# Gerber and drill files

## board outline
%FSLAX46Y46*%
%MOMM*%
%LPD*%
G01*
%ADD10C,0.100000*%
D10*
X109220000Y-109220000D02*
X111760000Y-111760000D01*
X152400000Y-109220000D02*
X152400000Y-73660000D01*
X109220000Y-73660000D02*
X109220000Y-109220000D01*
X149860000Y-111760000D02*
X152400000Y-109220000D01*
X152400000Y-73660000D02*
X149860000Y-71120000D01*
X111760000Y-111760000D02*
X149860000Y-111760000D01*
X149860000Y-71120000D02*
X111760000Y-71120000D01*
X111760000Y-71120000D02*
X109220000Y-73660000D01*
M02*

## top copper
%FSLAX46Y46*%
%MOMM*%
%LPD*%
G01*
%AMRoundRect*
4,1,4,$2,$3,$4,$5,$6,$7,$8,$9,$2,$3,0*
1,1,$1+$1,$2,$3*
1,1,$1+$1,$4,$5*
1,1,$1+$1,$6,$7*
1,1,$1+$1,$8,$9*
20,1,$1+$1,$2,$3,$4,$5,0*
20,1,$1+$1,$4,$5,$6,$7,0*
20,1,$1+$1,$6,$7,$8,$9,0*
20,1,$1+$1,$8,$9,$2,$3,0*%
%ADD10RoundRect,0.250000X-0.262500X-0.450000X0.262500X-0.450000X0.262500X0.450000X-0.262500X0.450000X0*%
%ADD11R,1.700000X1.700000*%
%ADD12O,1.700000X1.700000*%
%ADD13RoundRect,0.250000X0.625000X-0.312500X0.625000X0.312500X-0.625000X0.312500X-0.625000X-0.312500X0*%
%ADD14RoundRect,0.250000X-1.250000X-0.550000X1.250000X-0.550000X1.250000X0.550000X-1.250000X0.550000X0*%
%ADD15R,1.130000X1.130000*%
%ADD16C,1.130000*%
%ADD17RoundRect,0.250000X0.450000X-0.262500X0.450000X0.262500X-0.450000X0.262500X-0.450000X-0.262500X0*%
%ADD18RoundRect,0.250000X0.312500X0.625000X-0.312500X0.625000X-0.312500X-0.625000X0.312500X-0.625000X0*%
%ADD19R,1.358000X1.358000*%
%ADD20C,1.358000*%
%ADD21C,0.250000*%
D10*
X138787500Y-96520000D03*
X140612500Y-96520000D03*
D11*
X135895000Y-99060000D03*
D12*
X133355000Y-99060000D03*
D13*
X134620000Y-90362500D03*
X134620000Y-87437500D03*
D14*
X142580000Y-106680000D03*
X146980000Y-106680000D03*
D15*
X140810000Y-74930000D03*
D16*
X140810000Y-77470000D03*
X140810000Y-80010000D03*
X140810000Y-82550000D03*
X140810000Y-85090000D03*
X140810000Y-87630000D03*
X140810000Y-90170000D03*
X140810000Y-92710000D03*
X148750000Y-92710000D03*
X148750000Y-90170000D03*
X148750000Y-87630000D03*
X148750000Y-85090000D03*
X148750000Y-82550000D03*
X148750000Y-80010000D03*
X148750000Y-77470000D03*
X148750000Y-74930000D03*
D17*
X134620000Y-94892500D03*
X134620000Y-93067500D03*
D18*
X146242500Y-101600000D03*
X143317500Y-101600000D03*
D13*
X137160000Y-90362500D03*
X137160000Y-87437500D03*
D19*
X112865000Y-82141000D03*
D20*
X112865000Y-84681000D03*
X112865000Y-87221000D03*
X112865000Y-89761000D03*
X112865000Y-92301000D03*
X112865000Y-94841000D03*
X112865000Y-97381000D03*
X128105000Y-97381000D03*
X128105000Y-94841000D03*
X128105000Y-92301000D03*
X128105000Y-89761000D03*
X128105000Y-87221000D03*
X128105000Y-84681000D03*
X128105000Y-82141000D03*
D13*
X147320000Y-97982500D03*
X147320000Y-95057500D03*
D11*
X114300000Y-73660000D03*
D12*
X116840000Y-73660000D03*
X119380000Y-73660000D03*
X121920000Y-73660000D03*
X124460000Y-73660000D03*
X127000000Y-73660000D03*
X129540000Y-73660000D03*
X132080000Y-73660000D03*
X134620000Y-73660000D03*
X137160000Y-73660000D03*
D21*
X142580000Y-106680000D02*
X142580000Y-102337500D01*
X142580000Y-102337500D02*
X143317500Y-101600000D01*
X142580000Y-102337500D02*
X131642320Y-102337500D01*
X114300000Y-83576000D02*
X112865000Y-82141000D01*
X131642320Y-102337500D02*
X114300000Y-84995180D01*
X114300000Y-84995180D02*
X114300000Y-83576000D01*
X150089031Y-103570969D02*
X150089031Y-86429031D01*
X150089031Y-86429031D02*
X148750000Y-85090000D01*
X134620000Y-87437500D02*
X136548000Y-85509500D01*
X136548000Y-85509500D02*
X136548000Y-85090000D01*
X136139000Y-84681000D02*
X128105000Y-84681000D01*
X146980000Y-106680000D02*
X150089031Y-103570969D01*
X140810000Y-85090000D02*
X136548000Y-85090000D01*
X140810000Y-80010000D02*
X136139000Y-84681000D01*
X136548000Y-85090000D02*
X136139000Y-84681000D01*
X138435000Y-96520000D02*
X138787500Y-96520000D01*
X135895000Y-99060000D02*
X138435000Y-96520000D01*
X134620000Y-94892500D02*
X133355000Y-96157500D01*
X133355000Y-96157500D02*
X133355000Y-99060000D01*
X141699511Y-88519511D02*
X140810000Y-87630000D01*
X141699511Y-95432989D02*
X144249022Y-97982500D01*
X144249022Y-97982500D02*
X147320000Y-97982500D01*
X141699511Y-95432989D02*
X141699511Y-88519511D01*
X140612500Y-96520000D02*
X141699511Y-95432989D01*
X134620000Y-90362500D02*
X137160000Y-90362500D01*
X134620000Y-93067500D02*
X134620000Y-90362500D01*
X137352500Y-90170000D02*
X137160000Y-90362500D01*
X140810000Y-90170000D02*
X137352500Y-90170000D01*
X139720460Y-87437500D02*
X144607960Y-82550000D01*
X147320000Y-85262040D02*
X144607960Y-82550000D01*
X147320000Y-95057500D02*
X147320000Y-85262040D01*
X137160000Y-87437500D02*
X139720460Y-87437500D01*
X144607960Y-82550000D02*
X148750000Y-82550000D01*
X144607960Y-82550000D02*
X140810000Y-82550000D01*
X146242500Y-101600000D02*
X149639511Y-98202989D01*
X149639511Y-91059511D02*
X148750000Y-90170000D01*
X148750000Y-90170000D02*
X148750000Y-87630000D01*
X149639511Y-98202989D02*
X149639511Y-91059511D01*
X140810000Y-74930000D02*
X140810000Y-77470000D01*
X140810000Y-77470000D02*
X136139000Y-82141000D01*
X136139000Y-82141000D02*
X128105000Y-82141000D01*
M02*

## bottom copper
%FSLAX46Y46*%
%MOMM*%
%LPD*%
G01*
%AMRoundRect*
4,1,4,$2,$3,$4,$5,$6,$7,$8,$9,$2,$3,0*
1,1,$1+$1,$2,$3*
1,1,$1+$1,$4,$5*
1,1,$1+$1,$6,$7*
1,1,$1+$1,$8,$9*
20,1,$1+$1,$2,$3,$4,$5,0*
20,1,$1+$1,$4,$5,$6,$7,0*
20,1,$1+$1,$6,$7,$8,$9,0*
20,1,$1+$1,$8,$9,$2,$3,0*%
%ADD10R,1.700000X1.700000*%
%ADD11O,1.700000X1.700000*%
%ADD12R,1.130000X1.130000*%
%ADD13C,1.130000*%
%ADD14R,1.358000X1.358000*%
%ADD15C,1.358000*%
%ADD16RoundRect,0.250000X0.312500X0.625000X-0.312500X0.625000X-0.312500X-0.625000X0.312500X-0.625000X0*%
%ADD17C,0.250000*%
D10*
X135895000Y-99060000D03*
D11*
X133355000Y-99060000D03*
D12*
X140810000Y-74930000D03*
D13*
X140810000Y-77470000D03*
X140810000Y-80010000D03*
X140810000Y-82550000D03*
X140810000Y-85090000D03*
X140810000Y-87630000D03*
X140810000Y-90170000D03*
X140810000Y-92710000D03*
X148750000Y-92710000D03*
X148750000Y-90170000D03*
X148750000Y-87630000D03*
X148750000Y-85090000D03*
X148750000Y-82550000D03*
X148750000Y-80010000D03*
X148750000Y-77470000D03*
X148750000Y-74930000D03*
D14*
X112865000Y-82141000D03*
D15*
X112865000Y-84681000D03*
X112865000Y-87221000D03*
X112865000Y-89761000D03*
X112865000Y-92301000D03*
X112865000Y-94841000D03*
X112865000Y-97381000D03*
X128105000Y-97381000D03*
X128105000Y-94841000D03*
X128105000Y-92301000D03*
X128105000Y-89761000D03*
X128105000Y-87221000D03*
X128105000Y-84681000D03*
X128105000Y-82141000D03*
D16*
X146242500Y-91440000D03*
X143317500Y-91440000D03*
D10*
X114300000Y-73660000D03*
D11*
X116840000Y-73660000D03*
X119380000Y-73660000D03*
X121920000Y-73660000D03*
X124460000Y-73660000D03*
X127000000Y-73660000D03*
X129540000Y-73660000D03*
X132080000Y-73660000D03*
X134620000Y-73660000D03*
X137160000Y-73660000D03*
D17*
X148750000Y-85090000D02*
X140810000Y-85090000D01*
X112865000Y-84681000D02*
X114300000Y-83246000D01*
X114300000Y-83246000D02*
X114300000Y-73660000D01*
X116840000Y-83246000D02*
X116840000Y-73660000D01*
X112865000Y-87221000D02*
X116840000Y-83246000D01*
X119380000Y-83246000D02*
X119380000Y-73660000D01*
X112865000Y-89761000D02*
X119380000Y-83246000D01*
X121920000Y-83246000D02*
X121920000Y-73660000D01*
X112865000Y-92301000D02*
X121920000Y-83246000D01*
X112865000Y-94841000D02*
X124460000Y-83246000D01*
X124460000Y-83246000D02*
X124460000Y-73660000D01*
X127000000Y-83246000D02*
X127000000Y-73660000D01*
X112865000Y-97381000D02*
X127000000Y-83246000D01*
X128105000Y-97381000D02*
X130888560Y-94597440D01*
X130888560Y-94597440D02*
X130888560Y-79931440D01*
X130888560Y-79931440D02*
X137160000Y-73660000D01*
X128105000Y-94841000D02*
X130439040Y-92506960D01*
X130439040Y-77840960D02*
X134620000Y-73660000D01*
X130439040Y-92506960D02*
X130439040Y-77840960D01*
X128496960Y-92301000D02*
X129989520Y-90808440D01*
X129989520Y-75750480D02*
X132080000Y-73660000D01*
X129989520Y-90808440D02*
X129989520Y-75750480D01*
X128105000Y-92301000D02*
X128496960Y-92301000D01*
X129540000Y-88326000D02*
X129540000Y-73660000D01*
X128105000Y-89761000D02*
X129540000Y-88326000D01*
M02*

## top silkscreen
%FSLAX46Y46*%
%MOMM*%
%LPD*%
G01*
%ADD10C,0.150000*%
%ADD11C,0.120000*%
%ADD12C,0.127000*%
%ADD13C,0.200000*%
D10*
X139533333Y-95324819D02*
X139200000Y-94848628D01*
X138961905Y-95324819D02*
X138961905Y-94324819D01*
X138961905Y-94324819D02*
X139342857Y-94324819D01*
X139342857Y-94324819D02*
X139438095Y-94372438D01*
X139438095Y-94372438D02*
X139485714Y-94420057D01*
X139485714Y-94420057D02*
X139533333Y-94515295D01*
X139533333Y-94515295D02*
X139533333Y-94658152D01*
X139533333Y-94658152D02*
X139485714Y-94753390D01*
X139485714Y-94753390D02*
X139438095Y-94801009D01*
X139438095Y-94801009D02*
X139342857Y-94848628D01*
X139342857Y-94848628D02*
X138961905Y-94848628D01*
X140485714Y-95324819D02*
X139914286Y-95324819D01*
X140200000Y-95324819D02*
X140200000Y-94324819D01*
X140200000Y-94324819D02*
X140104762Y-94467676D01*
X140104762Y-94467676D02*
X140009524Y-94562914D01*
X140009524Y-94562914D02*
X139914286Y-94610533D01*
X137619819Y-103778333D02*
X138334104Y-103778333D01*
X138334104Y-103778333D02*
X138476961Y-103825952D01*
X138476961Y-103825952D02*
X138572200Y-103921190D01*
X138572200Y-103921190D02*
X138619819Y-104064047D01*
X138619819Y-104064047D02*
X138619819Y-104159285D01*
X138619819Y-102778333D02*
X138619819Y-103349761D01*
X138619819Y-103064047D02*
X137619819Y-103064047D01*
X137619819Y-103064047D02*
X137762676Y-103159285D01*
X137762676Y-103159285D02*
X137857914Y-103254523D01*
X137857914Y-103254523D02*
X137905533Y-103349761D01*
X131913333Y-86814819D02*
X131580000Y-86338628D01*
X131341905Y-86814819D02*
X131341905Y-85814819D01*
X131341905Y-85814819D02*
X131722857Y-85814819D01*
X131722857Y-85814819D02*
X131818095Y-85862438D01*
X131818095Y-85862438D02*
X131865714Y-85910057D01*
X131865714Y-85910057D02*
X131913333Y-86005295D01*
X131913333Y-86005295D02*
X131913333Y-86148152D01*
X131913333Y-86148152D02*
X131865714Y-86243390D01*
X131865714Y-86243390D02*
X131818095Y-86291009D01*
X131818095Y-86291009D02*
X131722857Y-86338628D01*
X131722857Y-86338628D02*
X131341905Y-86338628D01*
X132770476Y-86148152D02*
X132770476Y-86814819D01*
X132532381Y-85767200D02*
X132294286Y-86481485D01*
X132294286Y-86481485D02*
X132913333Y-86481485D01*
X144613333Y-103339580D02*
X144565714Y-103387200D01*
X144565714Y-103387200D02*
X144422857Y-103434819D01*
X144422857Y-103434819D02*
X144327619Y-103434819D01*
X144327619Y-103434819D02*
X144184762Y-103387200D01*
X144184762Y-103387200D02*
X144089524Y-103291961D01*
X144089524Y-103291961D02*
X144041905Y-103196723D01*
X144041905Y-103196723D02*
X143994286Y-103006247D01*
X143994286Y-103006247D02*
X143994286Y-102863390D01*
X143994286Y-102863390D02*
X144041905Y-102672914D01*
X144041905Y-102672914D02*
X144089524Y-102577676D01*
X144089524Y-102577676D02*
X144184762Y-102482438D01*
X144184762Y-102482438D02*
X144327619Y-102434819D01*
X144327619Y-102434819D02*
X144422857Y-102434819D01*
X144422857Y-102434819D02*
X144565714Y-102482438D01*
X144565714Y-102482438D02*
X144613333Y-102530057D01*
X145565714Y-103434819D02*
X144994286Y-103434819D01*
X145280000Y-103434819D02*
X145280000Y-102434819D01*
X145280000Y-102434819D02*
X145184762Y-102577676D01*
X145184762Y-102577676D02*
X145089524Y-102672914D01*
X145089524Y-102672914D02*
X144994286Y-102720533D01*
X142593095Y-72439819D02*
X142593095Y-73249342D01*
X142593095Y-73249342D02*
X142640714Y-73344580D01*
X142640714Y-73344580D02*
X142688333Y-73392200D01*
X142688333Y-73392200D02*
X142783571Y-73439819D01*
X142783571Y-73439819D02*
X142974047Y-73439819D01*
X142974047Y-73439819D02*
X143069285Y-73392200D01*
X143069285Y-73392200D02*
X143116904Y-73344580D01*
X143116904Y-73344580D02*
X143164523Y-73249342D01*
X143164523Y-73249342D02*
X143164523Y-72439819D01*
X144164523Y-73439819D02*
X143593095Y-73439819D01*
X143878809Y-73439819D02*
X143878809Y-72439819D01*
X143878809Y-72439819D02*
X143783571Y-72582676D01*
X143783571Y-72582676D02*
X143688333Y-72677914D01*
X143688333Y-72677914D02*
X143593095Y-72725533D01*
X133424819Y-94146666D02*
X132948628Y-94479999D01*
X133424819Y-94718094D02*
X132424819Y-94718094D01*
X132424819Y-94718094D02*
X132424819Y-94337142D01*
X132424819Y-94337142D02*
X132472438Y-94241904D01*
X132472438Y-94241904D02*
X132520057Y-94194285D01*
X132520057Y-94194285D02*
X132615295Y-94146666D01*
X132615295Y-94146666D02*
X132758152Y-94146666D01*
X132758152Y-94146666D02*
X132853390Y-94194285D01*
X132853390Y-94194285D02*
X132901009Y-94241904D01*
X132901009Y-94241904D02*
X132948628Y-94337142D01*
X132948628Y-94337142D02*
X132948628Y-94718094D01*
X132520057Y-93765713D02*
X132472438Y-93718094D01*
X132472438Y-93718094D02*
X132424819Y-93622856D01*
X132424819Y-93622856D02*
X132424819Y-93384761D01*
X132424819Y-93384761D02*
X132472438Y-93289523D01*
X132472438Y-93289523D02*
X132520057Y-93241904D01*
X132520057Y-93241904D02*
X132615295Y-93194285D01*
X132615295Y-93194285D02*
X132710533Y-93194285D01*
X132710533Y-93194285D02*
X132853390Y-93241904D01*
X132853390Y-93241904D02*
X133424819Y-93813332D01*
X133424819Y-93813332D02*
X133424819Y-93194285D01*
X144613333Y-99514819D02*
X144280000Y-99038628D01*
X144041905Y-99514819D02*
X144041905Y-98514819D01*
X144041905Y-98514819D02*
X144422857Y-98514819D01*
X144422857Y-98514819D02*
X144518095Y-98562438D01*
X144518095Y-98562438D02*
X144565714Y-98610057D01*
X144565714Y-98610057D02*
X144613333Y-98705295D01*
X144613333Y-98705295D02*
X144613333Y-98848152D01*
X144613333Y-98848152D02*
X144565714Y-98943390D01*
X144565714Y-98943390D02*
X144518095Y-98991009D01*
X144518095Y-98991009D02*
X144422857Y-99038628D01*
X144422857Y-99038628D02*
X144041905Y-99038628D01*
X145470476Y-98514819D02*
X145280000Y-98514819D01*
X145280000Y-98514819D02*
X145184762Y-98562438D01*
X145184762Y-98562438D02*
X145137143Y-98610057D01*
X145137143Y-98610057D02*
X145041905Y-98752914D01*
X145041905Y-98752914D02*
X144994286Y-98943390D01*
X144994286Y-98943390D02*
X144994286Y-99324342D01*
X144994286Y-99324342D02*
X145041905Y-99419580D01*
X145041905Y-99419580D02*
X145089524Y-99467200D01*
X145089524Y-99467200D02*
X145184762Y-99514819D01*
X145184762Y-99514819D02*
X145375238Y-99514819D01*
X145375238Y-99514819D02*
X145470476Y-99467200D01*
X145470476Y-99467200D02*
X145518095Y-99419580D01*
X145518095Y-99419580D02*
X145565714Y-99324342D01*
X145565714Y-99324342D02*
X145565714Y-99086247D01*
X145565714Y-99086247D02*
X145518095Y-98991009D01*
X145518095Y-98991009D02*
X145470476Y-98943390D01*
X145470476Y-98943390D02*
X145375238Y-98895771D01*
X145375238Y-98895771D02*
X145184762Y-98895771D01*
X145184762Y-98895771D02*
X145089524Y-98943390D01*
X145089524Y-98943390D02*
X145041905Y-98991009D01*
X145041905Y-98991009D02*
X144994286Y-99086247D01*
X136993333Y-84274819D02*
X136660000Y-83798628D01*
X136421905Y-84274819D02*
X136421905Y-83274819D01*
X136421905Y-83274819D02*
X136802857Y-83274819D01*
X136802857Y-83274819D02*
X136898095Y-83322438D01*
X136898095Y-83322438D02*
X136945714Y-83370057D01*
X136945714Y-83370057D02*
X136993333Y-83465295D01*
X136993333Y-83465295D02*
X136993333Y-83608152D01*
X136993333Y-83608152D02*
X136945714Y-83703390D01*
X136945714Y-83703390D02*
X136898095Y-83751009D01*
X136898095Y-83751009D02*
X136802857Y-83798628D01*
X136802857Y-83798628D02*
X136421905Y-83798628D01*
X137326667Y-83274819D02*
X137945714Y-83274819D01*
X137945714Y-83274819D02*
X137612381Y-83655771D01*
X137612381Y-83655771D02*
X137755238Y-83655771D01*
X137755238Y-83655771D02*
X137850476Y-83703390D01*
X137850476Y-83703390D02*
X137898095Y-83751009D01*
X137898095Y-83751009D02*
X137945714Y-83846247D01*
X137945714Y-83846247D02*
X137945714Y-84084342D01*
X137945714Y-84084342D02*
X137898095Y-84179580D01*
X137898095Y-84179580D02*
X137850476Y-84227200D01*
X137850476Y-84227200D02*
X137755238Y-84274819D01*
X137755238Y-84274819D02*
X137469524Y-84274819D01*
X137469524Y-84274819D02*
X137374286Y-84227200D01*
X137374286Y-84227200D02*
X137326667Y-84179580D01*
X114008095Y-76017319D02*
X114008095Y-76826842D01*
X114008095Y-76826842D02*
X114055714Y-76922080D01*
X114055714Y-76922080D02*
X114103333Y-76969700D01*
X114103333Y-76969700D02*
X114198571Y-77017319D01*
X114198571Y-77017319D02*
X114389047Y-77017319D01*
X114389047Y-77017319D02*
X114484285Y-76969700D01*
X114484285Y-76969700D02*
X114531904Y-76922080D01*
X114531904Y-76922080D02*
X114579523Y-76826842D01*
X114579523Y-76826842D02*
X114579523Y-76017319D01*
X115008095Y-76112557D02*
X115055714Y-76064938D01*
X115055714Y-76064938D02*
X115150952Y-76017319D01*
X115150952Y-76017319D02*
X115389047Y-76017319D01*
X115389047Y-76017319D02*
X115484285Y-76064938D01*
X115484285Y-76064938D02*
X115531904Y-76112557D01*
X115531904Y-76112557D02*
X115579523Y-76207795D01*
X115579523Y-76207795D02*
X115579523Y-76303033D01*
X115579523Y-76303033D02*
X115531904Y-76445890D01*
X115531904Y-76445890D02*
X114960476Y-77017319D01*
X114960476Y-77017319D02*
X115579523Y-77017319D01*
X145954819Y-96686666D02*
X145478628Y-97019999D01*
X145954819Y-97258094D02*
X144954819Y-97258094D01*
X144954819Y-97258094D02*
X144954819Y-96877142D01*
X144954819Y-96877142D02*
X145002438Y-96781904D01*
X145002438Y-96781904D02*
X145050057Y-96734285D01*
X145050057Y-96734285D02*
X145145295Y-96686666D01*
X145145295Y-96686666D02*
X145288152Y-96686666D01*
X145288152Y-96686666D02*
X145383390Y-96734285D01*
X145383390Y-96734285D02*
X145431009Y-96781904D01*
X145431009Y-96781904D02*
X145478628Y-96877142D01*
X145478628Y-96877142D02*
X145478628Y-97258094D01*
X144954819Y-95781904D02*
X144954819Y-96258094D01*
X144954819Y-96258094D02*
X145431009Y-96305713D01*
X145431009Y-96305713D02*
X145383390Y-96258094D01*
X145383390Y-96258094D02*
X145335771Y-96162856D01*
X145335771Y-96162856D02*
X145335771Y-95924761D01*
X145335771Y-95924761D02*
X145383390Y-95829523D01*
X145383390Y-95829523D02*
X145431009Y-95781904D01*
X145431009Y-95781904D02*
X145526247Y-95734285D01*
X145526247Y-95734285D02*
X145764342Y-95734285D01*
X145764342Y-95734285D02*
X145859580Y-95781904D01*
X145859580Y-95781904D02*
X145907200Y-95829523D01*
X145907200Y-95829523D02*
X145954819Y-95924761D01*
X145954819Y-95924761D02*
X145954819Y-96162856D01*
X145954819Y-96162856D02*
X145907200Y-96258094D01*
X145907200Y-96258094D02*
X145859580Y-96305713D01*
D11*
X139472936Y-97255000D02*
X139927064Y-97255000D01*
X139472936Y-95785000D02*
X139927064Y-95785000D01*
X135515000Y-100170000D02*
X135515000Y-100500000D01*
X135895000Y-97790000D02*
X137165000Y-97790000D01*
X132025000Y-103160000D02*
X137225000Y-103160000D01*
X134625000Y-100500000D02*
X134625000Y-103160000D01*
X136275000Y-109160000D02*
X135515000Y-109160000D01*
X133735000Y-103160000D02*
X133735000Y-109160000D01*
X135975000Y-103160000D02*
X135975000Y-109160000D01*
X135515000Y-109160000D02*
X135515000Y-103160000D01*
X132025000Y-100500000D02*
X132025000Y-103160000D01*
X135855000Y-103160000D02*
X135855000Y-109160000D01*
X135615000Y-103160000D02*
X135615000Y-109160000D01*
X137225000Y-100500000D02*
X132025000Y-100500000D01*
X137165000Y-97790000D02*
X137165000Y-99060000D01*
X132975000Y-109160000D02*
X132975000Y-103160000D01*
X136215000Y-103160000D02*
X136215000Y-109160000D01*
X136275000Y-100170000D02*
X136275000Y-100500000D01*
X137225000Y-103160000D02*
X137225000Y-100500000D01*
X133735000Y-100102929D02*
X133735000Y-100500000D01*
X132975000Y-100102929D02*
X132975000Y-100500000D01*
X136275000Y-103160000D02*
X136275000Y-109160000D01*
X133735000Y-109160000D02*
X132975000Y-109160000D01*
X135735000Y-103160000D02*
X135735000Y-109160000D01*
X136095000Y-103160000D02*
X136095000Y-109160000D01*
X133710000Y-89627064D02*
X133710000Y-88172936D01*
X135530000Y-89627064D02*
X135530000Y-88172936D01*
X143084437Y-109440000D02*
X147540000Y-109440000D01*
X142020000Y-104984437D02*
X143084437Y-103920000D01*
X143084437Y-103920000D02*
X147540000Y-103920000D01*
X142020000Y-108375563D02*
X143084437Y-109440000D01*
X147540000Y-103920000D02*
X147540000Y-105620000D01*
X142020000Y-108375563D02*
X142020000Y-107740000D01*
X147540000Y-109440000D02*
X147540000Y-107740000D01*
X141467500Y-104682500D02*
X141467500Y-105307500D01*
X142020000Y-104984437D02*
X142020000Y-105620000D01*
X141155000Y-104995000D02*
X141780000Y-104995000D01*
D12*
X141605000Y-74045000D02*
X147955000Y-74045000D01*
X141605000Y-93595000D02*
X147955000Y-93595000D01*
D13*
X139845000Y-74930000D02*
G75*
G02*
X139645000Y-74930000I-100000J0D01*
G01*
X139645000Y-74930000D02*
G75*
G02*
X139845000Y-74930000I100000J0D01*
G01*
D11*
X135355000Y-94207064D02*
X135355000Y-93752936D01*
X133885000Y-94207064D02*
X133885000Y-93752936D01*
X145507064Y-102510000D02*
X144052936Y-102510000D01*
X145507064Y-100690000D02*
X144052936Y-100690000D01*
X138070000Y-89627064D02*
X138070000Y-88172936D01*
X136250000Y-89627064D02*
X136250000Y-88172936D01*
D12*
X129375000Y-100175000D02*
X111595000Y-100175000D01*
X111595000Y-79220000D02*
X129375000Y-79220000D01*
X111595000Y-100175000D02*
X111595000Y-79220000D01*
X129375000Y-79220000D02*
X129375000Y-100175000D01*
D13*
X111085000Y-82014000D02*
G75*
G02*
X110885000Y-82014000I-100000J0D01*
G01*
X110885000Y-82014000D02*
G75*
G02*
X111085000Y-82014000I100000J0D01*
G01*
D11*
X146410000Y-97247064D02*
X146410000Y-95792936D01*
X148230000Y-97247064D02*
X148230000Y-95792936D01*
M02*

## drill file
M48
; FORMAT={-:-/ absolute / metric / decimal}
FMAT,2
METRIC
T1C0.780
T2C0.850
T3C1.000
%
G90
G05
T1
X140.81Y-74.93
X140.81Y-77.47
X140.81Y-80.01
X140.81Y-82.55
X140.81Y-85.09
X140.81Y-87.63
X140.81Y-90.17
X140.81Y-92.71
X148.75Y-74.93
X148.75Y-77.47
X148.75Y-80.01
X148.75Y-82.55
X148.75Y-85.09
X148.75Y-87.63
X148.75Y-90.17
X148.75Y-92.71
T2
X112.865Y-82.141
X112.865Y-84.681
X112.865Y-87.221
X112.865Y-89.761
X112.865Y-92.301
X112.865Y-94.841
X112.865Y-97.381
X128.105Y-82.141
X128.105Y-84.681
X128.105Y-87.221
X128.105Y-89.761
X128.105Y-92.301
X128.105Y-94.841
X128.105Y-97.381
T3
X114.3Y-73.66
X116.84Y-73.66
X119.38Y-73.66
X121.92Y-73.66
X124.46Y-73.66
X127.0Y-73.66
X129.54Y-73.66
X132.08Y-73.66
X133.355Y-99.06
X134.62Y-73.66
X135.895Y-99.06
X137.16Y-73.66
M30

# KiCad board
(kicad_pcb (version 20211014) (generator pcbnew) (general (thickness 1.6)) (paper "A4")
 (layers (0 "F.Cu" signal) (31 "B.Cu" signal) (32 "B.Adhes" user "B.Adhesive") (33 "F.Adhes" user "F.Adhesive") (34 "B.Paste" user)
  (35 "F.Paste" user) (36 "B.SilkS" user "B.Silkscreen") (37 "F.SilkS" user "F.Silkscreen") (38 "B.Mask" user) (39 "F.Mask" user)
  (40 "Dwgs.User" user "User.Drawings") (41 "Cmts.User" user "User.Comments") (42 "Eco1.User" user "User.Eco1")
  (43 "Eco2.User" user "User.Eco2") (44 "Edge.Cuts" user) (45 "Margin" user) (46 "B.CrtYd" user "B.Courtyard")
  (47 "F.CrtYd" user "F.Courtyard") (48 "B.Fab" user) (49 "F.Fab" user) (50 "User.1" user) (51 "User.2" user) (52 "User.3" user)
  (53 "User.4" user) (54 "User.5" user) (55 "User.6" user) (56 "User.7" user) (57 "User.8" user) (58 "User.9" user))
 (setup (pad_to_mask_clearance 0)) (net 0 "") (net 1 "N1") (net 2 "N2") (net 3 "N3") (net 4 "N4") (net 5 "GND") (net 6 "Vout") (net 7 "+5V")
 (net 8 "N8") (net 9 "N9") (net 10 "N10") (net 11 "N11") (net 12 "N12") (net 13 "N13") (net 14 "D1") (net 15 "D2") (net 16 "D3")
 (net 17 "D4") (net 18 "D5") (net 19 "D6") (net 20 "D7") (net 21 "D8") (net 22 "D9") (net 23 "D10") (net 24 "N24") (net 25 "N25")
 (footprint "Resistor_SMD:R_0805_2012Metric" (layer "F.Cu") (at 139.7 96.52)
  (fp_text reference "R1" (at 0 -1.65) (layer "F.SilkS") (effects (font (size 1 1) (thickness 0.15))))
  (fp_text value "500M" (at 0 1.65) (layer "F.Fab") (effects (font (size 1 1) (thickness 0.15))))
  (fp_line (start -0.227064 0.735) (end 0.227064 0.735) (layer "F.SilkS") (width 0.12))
  (fp_line (start -0.227064 -0.735) (end 0.227064 -0.735) (layer "F.SilkS") (width 0.12))
  (pad "1" smd roundrect (at -0.9125 0) (size 1.025 1.4) (layers "F.Cu" "F.Paste" "F.Mask") (roundrect_rratio 0.243902) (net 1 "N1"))
  (pad "2" smd roundrect (at 0.9125 0) (size 1.025 1.4) (layers "F.Cu" "F.Paste" "F.Mask") (roundrect_rratio 0.243902) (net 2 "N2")))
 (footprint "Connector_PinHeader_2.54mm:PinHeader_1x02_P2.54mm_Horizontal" (layer "F.Cu") (at 135.895 99.06 -90)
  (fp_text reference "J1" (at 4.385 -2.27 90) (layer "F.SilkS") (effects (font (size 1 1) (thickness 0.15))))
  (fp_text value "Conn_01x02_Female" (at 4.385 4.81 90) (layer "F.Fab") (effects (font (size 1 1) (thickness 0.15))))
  (fp_line (start 1.11 0.38) (end 1.44 0.38) (layer "F.SilkS") (width 0.12))
  (fp_line (start -1.27 0) (end -1.27 -1.27) (layer "F.SilkS") (width 0.12))
  (fp_line (start 4.1 3.87) (end 4.1 -1.33) (layer "F.SilkS") (width 0.12))
  (fp_line (start 1.44 1.27) (end 4.1 1.27) (layer "F.SilkS") (width 0.12))
  (fp_line (start 10.1 -0.38) (end 10.1 0.38) (layer "F.SilkS") (width 0.12))
  (fp_line (start 4.1 2.16) (end 10.1 2.16) (layer "F.SilkS") (width 0.12))
  (fp_line (start 4.1 -0.08) (end 10.1 -0.08) (layer "F.SilkS") (width 0.12))
  (fp_line (start 10.1 0.38) (end 4.1 0.38) (layer "F.SilkS") (width 0.12))
  (fp_line (start 1.44 3.87) (end 4.1 3.87) (layer "F.SilkS") (width 0.12))
  (fp_line (start 4.1 0.04) (end 10.1 0.04) (layer "F.SilkS") (width 0.12))
  (fp_line (start 4.1 0.28) (end 10.1 0.28) (layer "F.SilkS") (width 0.12))
  (fp_line (start 1.44 -1.33) (end 1.44 3.87) (layer "F.SilkS") (width 0.12))
  (fp_line (start -1.27 -1.27) (end 0 -1.27) (layer "F.SilkS") (width 0.12))
  (fp_line (start 10.1 2.92) (end 4.1 2.92) (layer "F.SilkS") (width 0.12))
  (fp_line (start 4.1 -0.32) (end 10.1 -0.32) (layer "F.SilkS") (width 0.12))
  (fp_line (start 1.11 -0.38) (end 1.44 -0.38) (layer "F.SilkS") (width 0.12))
  (fp_line (start 4.1 -1.33) (end 1.44 -1.33) (layer "F.SilkS") (width 0.12))
  (fp_line (start 1.042929 2.16) (end 1.44 2.16) (layer "F.SilkS") (width 0.12))
  (fp_line (start 1.042929 2.92) (end 1.44 2.92) (layer "F.SilkS") (width 0.12))
  (fp_line (start 4.1 -0.38) (end 10.1 -0.38) (layer "F.SilkS") (width 0.12))
  (fp_line (start 10.1 2.16) (end 10.1 2.92) (layer "F.SilkS") (width 0.12))
  (fp_line (start 4.1 0.16) (end 10.1 0.16) (layer "F.SilkS") (width 0.12))
  (fp_line (start 4.1 -0.2) (end 10.1 -0.2) (layer "F.SilkS") (width 0.12))
  (pad "1" thru_hole rect (at 0 0 270) (size 1.7 1.7) (drill 1) (layers *.Cu *.Mask) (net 1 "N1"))
  (pad "2" thru_hole oval (at 0 2.54 270) (size 1.7 1.7) (drill 1) (layers *.Cu *.Mask) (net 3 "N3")))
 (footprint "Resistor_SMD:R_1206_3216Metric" (layer "F.Cu") (at 134.62 88.9 90)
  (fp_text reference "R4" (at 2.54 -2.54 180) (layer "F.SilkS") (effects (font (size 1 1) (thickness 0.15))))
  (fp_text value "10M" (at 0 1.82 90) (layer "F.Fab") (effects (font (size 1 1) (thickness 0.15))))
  (fp_line (start -0.727064 -0.91) (end 0.727064 -0.91) (layer "F.SilkS") (width 0.12))
  (fp_line (start -0.727064 0.91) (end 0.727064 0.91) (layer "F.SilkS") (width 0.12))
  (pad "1" smd roundrect (at -1.4625 0 90) (size 1.125 1.75) (layers "F.Cu" "F.Paste" "F.Mask") (roundrect_rratio 0.222222) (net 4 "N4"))
  (pad "2" smd roundrect (at 1.4625 0 90) (size 1.125 1.75) (layers "F.Cu" "F.Paste" "F.Mask") (roundrect_rratio 0.222222) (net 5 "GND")))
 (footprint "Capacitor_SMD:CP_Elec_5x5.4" (layer "F.Cu") (at 144.78 106.68)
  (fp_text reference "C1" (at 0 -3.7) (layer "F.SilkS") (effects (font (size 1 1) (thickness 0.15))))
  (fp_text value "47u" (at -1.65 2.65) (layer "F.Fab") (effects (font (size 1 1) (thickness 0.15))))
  (fp_line (start -1.695563 2.76) (end 2.76 2.76) (layer "F.SilkS") (width 0.12))
  (fp_line (start -2.76 -1.695563) (end -1.695563 -2.76) (layer "F.SilkS") (width 0.12))
  (fp_line (start -1.695563 -2.76) (end 2.76 -2.76) (layer "F.SilkS") (width 0.12))
  (fp_line (start -2.76 1.695563) (end -1.695563 2.76) (layer "F.SilkS") (width 0.12))
  (fp_line (start 2.76 -2.76) (end 2.76 -1.06) (layer "F.SilkS") (width 0.12))
  (fp_line (start -2.76 1.695563) (end -2.76 1.06) (layer "F.SilkS") (width 0.12))
  (fp_line (start 2.76 2.76) (end 2.76 1.06) (layer "F.SilkS") (width 0.12))
  (fp_line (start -3.3125 -1.9975) (end -3.3125 -1.3725) (layer "F.SilkS") (width 0.12))
  (fp_line (start -2.76 -1.695563) (end -2.76 -1.06) (layer "F.SilkS") (width 0.12))
  (fp_line (start -3.625 -1.685) (end -3 -1.685) (layer "F.SilkS") (width 0.12))
  (pad "1" smd roundrect (at -2.2 0) (size 3 1.6) (layers "F.Cu" "F.Paste" "F.Mask") (roundrect_rratio 0.15625) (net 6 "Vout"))
  (pad "2" smd roundrect (at 2.2 0) (size 3 1.6) (layers "F.Cu" "F.Paste" "F.Mask") (roundrect_rratio 0.15625) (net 5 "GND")))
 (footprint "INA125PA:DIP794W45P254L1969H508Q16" (layer "F.Cu") (at 144.78 83.82)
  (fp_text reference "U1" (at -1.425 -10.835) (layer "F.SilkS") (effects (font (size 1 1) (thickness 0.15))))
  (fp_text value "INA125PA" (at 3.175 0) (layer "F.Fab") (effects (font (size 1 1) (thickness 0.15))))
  (fp_line (start -3.175 -9.775) (end 3.175 -9.775) (layer "F.SilkS") (width 0.127))
  (fp_line (start -3.175 9.775) (end 3.175 9.775) (layer "F.SilkS") (width 0.127))
  (fp_circle (center -5.035 -8.89) (end -4.935 -8.89) (layer "F.SilkS") (width 0.2) (fill none))
  (pad "1" thru_hole rect locked (at -3.97 -8.89) (size 1.13 1.13) (drill 0.78) (layers *.Cu *.Mask) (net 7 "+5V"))
  (pad "2" thru_hole circle locked (at -3.97 -6.35) (size 1.13 1.13) (drill 0.78) (layers *.Cu *.Mask) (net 7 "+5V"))
  (pad "3" thru_hole circle locked (at -3.97 -3.81) (size 1.13 1.13) (drill 0.78) (layers *.Cu *.Mask) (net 5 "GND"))
  (pad "4" thru_hole circle locked (at -3.97 -1.27) (size 1.13 1.13) (drill 0.78) (layers *.Cu *.Mask) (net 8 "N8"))
  (pad "5" thru_hole circle locked (at -3.97 1.27) (size 1.13 1.13) (drill 0.78) (layers *.Cu *.Mask) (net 5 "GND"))
  (pad "6" thru_hole circle locked (at -3.97 3.81) (size 1.13 1.13) (drill 0.78) (layers *.Cu *.Mask) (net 2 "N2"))
  (pad "7" thru_hole circle locked (at -3.97 6.35) (size 1.13 1.13) (drill 0.78) (layers *.Cu *.Mask) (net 4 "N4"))
  (pad "8" thru_hole circle locked (at -3.97 8.89) (size 1.13 1.13) (drill 0.78) (layers *.Cu *.Mask) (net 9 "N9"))
  (pad "9" thru_hole circle locked (at 3.97 8.89) (size 1.13 1.13) (drill 0.78) (layers *.Cu *.Mask) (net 9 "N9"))
  (pad "10" thru_hole circle locked (at 3.97 6.35) (size 1.13 1.13) (drill 0.78) (layers *.Cu *.Mask) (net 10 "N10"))
  (pad "11" thru_hole circle locked (at 3.97 3.81) (size 1.13 1.13) (drill 0.78) (layers *.Cu *.Mask) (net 10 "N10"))
  (pad "12" thru_hole circle locked (at 3.97 1.27) (size 1.13 1.13) (drill 0.78) (layers *.Cu *.Mask) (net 5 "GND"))
  (pad "13" thru_hole circle locked (at 3.97 -1.27) (size 1.13 1.13) (drill 0.78) (layers *.Cu *.Mask) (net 8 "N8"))
  (pad "14" thru_hole circle locked (at 3.97 -3.81) (size 1.13 1.13) (drill 0.78) (layers *.Cu *.Mask) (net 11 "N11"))
  (pad "15" thru_hole circle locked (at 3.97 -6.35) (size 1.13 1.13) (drill 0.78) (layers *.Cu *.Mask) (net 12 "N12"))
  (pad "16" thru_hole circle locked (at 3.97 -8.89) (size 1.13 1.13) (drill 0.78) (layers *.Cu *.Mask) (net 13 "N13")))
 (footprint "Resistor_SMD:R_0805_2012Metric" (layer "F.Cu") (at 134.62 93.98 90)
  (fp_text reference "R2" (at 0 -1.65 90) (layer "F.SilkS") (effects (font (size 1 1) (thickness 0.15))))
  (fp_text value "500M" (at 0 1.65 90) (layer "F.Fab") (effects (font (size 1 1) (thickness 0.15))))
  (fp_line (start -0.227064 0.735) (end 0.227064 0.735) (layer "F.SilkS") (width 0.12))
  (fp_line (start -0.227064 -0.735) (end 0.227064 -0.735) (layer "F.SilkS") (width 0.12))
  (pad "1" smd roundrect (at -0.9125 0 90) (size 1.025 1.4) (layers "F.Cu" "F.Paste" "F.Mask") (roundrect_rratio 0.243902) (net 3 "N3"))
  (pad "2" smd roundrect (at 0.9125 0 90) (size 1.025 1.4) (layers "F.Cu" "F.Paste" "F.Mask") (roundrect_rratio 0.243902) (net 4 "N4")))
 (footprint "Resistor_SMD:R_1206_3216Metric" (layer "F.Cu") (at 144.78 101.6 180)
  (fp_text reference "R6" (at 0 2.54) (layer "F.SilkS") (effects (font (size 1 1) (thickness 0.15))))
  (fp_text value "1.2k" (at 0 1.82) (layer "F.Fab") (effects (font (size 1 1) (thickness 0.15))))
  (fp_line (start -0.727064 -0.91) (end 0.727064 -0.91) (layer "F.SilkS") (width 0.12))
  (fp_line (start -0.727064 0.91) (end 0.727064 0.91) (layer "F.SilkS") (width 0.12))
  (pad "1" smd roundrect (at -1.4625 0 180) (size 1.125 1.75) (layers "F.Cu" "F.Paste" "F.Mask") (roundrect_rratio 0.222222) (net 10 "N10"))
  (pad "2" smd roundrect (at 1.4625 0 180) (size 1.125 1.75) (layers "F.Cu" "F.Paste" "F.Mask") (roundrect_rratio 0.222222) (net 6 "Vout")))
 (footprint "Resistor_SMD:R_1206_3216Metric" (layer "F.Cu") (at 137.16 88.9 90)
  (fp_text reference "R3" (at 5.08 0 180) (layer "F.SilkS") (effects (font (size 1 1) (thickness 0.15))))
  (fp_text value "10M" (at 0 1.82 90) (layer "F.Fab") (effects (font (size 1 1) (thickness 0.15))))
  (fp_line (start -0.727064 0.91) (end 0.727064 0.91) (layer "F.SilkS") (width 0.12))
  (fp_line (start -0.727064 -0.91) (end 0.727064 -0.91) (layer "F.SilkS") (width 0.12))
  (pad "1" smd roundrect (at -1.4625 0 90) (size 1.125 1.75) (layers "F.Cu" "F.Paste" "F.Mask") (roundrect_rratio 0.222222) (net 4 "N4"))
  (pad "2" smd roundrect (at 1.4625 0 90) (size 1.125 1.75) (layers "F.Cu" "F.Paste" "F.Mask") (roundrect_rratio 0.222222) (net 8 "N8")))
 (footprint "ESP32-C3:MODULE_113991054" (layer "F.Cu") (at 120.485 89.6975)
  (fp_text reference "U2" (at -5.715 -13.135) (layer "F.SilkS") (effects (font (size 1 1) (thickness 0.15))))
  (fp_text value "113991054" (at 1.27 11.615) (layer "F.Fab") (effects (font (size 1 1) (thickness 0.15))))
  (fp_line (start 8.89 10.4775) (end -8.89 10.4775) (layer "F.SilkS") (width 0.127))
  (fp_line (start -8.89 -10.4775) (end 8.89 -10.4775) (layer "F.SilkS") (width 0.127))
  (fp_line (start -8.89 10.4775) (end -8.89 -10.4775) (layer "F.SilkS") (width 0.127))
  (fp_line (start 8.89 -10.4775) (end 8.89 10.4775) (layer "F.SilkS") (width 0.127))
  (fp_circle (center -9.5 -7.6835) (end -9.4 -7.6835) (layer "F.SilkS") (width 0.2) (fill none))
  (pad "1" thru_hole rect locked (at -7.62 -7.5565) (size 1.358 1.358) (drill 0.85) (layers *.Cu *.Mask) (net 6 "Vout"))
  (pad "2" thru_hole circle locked (at -7.62 -5.0165) (size 1.358 1.358) (drill 0.85) (layers *.Cu *.Mask) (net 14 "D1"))
  (pad "3" thru_hole circle locked (at -7.62 -2.4765) (size 1.358 1.358) (drill 0.85) (layers *.Cu *.Mask) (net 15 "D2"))
  (pad "4" thru_hole circle locked (at -7.62 0.0635) (size 1.358 1.358) (drill 0.85) (layers *.Cu *.Mask) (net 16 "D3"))
  (pad "5" thru_hole circle locked (at -7.62 2.6035) (size 1.358 1.358) (drill 0.85) (layers *.Cu *.Mask) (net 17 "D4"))
  (pad "6" thru_hole circle locked (at -7.62 5.1435) (size 1.358 1.358) (drill 0.85) (layers *.Cu *.Mask) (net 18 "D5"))
  (pad "7" thru_hole circle locked (at -7.62 7.6835) (size 1.358 1.358) (drill 0.85) (layers *.Cu *.Mask) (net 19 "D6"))
  (pad "8" thru_hole circle locked (at 7.62 7.6835) (size 1.358 1.358) (drill 0.85) (layers *.Cu *.Mask) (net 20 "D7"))
  (pad "9" thru_hole circle locked (at 7.62 5.1435) (size 1.358 1.358) (drill 0.85) (layers *.Cu *.Mask) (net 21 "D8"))
  (pad "10" thru_hole circle locked (at 7.62 2.6035) (size 1.358 1.358) (drill 0.85) (layers *.Cu *.Mask) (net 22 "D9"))
  (pad "11" thru_hole circle locked (at 7.62 0.0635) (size 1.358 1.358) (drill 0.85) (layers *.Cu *.Mask) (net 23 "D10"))
  (pad "12" thru_hole circle locked (at 7.62 -2.4765) (size 1.358 1.358) (drill 0.85) (layers *.Cu *.Mask) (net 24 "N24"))
  (pad "13" thru_hole circle locked (at 7.62 -5.0165) (size 1.358 1.358) (drill 0.85) (layers *.Cu *.Mask) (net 5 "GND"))
  (pad "14" thru_hole circle locked (at 7.62 -7.5565) (size 1.358 1.358) (drill 0.85) (layers *.Cu *.Mask) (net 7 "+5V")))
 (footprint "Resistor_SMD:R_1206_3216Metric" (layer "F.Cu") (at 147.32 96.52 90)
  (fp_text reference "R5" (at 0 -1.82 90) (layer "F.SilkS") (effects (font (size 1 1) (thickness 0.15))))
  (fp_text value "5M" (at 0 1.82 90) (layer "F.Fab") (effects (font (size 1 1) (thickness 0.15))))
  (fp_line (start -0.727064 -0.91) (end 0.727064 -0.91) (layer "F.SilkS") (width 0.12))
  (fp_line (start -0.727064 0.91) (end 0.727064 0.91) (layer "F.SilkS") (width 0.12))
  (pad "1" smd roundrect (at -1.4625 0 90) (size 1.125 1.75) (layers "F.Cu" "F.Paste" "F.Mask") (roundrect_rratio 0.222222) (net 2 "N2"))
  (pad "2" smd roundrect (at 1.4625 0 90) (size 1.125 1.75) (layers "F.Cu" "F.Paste" "F.Mask") (roundrect_rratio 0.222222) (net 8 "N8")))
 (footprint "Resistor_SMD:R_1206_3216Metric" (layer "B.Cu") (at 144.78 91.44 180)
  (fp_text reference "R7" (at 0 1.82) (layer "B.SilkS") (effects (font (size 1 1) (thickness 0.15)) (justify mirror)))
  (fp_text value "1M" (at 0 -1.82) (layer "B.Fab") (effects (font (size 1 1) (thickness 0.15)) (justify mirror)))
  (pad "1" smd roundrect (at -1.4625 0 180) (size 1.125 1.75) (layers "B.Cu" "B.Paste" "B.Mask") (roundrect_rratio 0.222222) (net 9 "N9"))
  (pad "2" smd roundrect (at 1.4625 0 180) (size 1.125 1.75) (layers "B.Cu" "B.Paste" "B.Mask") (roundrect_rratio 0.222222) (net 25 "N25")))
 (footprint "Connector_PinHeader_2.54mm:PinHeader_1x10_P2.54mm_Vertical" (layer "B.Cu") (at 114.3 73.66 -90)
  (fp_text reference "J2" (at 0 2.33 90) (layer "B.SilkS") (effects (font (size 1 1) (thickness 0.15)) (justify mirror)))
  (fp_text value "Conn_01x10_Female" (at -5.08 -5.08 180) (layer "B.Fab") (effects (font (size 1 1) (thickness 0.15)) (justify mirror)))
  (pad "1" thru_hole rect (at 0 0 270) (size 1.7 1.7) (drill 1) (layers *.Cu *.Mask) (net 14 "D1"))
  (pad "2" thru_hole oval (at 0 -2.54 270) (size 1.7 1.7) (drill 1) (layers *.Cu *.Mask) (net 15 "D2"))
  (pad "3" thru_hole oval (at 0 -5.08 270) (size 1.7 1.7) (drill 1) (layers *.Cu *.Mask) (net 16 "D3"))
  (pad "4" thru_hole oval (at 0 -7.62 270) (size 1.7 1.7) (drill 1) (layers *.Cu *.Mask) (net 17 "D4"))
  (pad "5" thru_hole oval (at 0 -10.16 270) (size 1.7 1.7) (drill 1) (layers *.Cu *.Mask) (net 18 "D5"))
  (pad "6" thru_hole oval (at 0 -12.7 270) (size 1.7 1.7) (drill 1) (layers *.Cu *.Mask) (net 19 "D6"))
  (pad "7" thru_hole oval (at 0 -15.24 270) (size 1.7 1.7) (drill 1) (layers *.Cu *.Mask) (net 23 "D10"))
  (pad "8" thru_hole oval (at 0 -17.78 270) (size 1.7 1.7) (drill 1) (layers *.Cu *.Mask) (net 22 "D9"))
  (pad "9" thru_hole oval (at 0 -20.32 270) (size 1.7 1.7) (drill 1) (layers *.Cu *.Mask) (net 21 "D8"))
  (pad "10" thru_hole oval (at 0 -22.86 270) (size 1.7 1.7) (drill 1) (layers *.Cu *.Mask) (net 20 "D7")))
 (gr_line (start 109.22 109.22) (end 111.76 111.76) (layer "Edge.Cuts") (width 0.1))
 (gr_line (start 152.4 109.22) (end 152.4 73.66) (layer "Edge.Cuts") (width 0.1))
 (gr_line (start 109.22 73.66) (end 109.22 109.22) (layer "Edge.Cuts") (width 0.1))
 (gr_line (start 149.86 111.76) (end 152.4 109.22) (layer "Edge.Cuts") (width 0.1))
 (gr_line (start 152.4 73.66) (end 149.86 71.12) (layer "Edge.Cuts") (width 0.1))
 (gr_line (start 111.76 111.76) (end 149.86 111.76) (layer "Edge.Cuts") (width 0.1))
 (gr_line (start 149.86 71.12) (end 111.76 71.12) (layer "Edge.Cuts") (width 0.1))
 (gr_line (start 111.76 71.12) (end 109.22 73.66) (layer "Edge.Cuts") (width 0.1))
 (segment (start 142.58 106.68) (end 142.58 102.3375) (width 0.25) (layer "F.Cu") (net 6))
 (segment (start 142.58 102.3375) (end 143.3175 101.6) (width 0.25) (layer "F.Cu") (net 6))
 (segment (start 142.58 102.3375) (end 131.64232 102.3375) (width 0.25) (layer "F.Cu") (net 6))
 (segment (start 114.3 83.576) (end 112.865 82.141) (width 0.25) (layer "F.Cu") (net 6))
 (segment (start 131.64232 102.3375) (end 114.3 84.99518) (width 0.25) (layer "F.Cu") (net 6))
 (segment (start 114.3 84.99518) (end 114.3 83.576) (width 0.25) (layer "F.Cu") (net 6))
 (segment (start 150.089031 103.570969) (end 150.089031 86.429031) (width 0.25) (layer "F.Cu") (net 5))
 (segment (start 150.089031 86.429031) (end 148.75 85.09) (width 0.25) (layer "F.Cu") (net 5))
 (segment (start 134.62 87.4375) (end 136.548 85.5095) (width 0.25) (layer "F.Cu") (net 5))
 (segment (start 136.548 85.5095) (end 136.548 85.09) (width 0.25) (layer "F.Cu") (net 5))
 (segment (start 136.139 84.681) (end 128.105 84.681) (width 0.25) (layer "F.Cu") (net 5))
 (segment (start 146.98 106.68) (end 150.089031 103.570969) (width 0.25) (layer "F.Cu") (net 5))
 (segment (start 140.81 85.09) (end 136.548 85.09) (width 0.25) (layer "F.Cu") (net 5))
 (segment (start 140.81 80.01) (end 136.139 84.681) (width 0.25) (layer "F.Cu") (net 5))
 (segment (start 136.548 85.09) (end 136.139 84.681) (width 0.25) (layer "F.Cu") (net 5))
 (segment (start 148.75 85.09) (end 140.81 85.09) (width 0.25) (layer "B.Cu") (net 5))
 (segment (start 138.435 96.52) (end 138.7875 96.52) (width 0.25) (layer "F.Cu") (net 1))
 (segment (start 135.895 99.06) (end 138.435 96.52) (width 0.25) (layer "F.Cu") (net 1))
 (segment (start 134.62 94.8925) (end 133.355 96.1575) (width 0.25) (layer "F.Cu") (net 3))
 (segment (start 133.355 96.1575) (end 133.355 99.06) (width 0.25) (layer "F.Cu") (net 3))
 (segment (start 112.865 84.681) (end 114.3 83.246) (width 0.25) (layer "B.Cu") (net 14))
 (segment (start 114.3 83.246) (end 114.3 73.66) (width 0.25) (layer "B.Cu") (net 14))
 (segment (start 116.84 83.246) (end 116.84 73.66) (width 0.25) (layer "B.Cu") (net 15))
 (segment (start 112.865 87.221) (end 116.84 83.246) (width 0.25) (layer "B.Cu") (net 15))
 (segment (start 119.38 83.246) (end 119.38 73.66) (width 0.25) (layer "B.Cu") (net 16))
 (segment (start 112.865 89.761) (end 119.38 83.246) (width 0.25) (layer "B.Cu") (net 16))
 (segment (start 121.92 83.246) (end 121.92 73.66) (width 0.25) (layer "B.Cu") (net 17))
 (segment (start 112.865 92.301) (end 121.92 83.246) (width 0.25) (layer "B.Cu") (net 17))
 (segment (start 112.865 94.841) (end 124.46 83.246) (width 0.25) (layer "B.Cu") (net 18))
 (segment (start 124.46 83.246) (end 124.46 73.66) (width 0.25) (layer "B.Cu") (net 18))
 (segment (start 127 83.246) (end 127 73.66) (width 0.25) (layer "B.Cu") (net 19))
 (segment (start 112.865 97.381) (end 127 83.246) (width 0.25) (layer "B.Cu") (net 19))
 (segment (start 128.105 97.381) (end 130.88856 94.59744) (width 0.25) (layer "B.Cu") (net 20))
 (segment (start 130.88856 94.59744) (end 130.88856 79.93144) (width 0.25) (layer "B.Cu") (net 20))
 (segment (start 130.88856 79.93144) (end 137.16 73.66) (width 0.25) (layer "B.Cu") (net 20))
 (segment (start 128.105 94.841) (end 130.43904 92.50696) (width 0.25) (layer "B.Cu") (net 21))
 (segment (start 130.43904 77.84096) (end 134.62 73.66) (width 0.25) (layer "B.Cu") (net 21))
 (segment (start 130.43904 92.50696) (end 130.43904 77.84096) (width 0.25) (layer "B.Cu") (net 21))
 (segment (start 128.49696 92.301) (end 129.98952 90.80844) (width 0.25) (layer "B.Cu") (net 22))
 (segment (start 129.98952 75.75048) (end 132.08 73.66) (width 0.25) (layer "B.Cu") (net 22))
 (segment (start 129.98952 90.80844) (end 129.98952 75.75048) (width 0.25) (layer "B.Cu") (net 22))
 (segment (start 128.105 92.301) (end 128.49696 92.301) (width 0.25) (layer "B.Cu") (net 22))
 (segment (start 129.54 88.326) (end 129.54 73.66) (width 0.25) (layer "B.Cu") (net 23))
 (segment (start 128.105 89.761) (end 129.54 88.326) (width 0.25) (layer "B.Cu") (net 23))
 (segment (start 141.699511 88.519511) (end 140.81 87.63) (width 0.25) (layer "F.Cu") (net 2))
 (segment (start 141.699511 95.432989) (end 144.249022 97.9825) (width 0.25) (layer "F.Cu") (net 2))
 (segment (start 144.249022 97.9825) (end 147.32 97.9825) (width 0.25) (layer "F.Cu") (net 2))
 (segment (start 141.699511 95.432989) (end 141.699511 88.519511) (width 0.25) (layer "F.Cu") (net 2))
 (segment (start 140.6125 96.52) (end 141.699511 95.432989) (width 0.25) (layer "F.Cu") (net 2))
 (segment (start 134.62 90.3625) (end 137.16 90.3625) (width 0.25) (layer "F.Cu") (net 4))
 (segment (start 134.62 93.0675) (end 134.62 90.3625) (width 0.25) (layer "F.Cu") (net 4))
 (segment (start 137.3525 90.17) (end 137.16 90.3625) (width 0.25) (layer "F.Cu") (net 4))
 (segment (start 140.81 90.17) (end 137.3525 90.17) (width 0.25) (layer "F.Cu") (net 4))
 (segment (start 139.72046 87.4375) (end 144.60796 82.55) (width 0.25) (layer "F.Cu") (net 8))
 (segment (start 147.32 85.26204) (end 144.60796 82.55) (width 0.25) (layer "F.Cu") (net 8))
 (segment (start 147.32 95.0575) (end 147.32 85.26204) (width 0.25) (layer "F.Cu") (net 8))
 (segment (start 137.16 87.4375) (end 139.72046 87.4375) (width 0.25) (layer "F.Cu") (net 8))
 (segment (start 144.60796 82.55) (end 148.75 82.55) (width 0.25) (layer "F.Cu") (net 8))
 (segment (start 144.60796 82.55) (end 140.81 82.55) (width 0.25) (layer "F.Cu") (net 8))
 (segment (start 146.2425 101.6) (end 149.639511 98.202989) (width 0.25) (layer "F.Cu") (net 10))
 (segment (start 149.639511 91.059511) (end 148.75 90.17) (width 0.25) (layer "F.Cu") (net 10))
 (segment (start 148.75 90.17) (end 148.75 87.63) (width 0.25) (layer "F.Cu") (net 10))
 (segment (start 149.639511 98.202989) (end 149.639511 91.059511) (width 0.25) (layer "F.Cu") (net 10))
 (segment (start 140.81 74.93) (end 140.81 77.47) (width 0.25) (layer "F.Cu") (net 7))
 (segment (start 140.81 77.47) (end 136.139 82.141) (width 0.25) (layer "F.Cu") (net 7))
 (segment (start 136.139 82.141) (end 128.105 82.141) (width 0.25) (layer "F.Cu") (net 7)))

